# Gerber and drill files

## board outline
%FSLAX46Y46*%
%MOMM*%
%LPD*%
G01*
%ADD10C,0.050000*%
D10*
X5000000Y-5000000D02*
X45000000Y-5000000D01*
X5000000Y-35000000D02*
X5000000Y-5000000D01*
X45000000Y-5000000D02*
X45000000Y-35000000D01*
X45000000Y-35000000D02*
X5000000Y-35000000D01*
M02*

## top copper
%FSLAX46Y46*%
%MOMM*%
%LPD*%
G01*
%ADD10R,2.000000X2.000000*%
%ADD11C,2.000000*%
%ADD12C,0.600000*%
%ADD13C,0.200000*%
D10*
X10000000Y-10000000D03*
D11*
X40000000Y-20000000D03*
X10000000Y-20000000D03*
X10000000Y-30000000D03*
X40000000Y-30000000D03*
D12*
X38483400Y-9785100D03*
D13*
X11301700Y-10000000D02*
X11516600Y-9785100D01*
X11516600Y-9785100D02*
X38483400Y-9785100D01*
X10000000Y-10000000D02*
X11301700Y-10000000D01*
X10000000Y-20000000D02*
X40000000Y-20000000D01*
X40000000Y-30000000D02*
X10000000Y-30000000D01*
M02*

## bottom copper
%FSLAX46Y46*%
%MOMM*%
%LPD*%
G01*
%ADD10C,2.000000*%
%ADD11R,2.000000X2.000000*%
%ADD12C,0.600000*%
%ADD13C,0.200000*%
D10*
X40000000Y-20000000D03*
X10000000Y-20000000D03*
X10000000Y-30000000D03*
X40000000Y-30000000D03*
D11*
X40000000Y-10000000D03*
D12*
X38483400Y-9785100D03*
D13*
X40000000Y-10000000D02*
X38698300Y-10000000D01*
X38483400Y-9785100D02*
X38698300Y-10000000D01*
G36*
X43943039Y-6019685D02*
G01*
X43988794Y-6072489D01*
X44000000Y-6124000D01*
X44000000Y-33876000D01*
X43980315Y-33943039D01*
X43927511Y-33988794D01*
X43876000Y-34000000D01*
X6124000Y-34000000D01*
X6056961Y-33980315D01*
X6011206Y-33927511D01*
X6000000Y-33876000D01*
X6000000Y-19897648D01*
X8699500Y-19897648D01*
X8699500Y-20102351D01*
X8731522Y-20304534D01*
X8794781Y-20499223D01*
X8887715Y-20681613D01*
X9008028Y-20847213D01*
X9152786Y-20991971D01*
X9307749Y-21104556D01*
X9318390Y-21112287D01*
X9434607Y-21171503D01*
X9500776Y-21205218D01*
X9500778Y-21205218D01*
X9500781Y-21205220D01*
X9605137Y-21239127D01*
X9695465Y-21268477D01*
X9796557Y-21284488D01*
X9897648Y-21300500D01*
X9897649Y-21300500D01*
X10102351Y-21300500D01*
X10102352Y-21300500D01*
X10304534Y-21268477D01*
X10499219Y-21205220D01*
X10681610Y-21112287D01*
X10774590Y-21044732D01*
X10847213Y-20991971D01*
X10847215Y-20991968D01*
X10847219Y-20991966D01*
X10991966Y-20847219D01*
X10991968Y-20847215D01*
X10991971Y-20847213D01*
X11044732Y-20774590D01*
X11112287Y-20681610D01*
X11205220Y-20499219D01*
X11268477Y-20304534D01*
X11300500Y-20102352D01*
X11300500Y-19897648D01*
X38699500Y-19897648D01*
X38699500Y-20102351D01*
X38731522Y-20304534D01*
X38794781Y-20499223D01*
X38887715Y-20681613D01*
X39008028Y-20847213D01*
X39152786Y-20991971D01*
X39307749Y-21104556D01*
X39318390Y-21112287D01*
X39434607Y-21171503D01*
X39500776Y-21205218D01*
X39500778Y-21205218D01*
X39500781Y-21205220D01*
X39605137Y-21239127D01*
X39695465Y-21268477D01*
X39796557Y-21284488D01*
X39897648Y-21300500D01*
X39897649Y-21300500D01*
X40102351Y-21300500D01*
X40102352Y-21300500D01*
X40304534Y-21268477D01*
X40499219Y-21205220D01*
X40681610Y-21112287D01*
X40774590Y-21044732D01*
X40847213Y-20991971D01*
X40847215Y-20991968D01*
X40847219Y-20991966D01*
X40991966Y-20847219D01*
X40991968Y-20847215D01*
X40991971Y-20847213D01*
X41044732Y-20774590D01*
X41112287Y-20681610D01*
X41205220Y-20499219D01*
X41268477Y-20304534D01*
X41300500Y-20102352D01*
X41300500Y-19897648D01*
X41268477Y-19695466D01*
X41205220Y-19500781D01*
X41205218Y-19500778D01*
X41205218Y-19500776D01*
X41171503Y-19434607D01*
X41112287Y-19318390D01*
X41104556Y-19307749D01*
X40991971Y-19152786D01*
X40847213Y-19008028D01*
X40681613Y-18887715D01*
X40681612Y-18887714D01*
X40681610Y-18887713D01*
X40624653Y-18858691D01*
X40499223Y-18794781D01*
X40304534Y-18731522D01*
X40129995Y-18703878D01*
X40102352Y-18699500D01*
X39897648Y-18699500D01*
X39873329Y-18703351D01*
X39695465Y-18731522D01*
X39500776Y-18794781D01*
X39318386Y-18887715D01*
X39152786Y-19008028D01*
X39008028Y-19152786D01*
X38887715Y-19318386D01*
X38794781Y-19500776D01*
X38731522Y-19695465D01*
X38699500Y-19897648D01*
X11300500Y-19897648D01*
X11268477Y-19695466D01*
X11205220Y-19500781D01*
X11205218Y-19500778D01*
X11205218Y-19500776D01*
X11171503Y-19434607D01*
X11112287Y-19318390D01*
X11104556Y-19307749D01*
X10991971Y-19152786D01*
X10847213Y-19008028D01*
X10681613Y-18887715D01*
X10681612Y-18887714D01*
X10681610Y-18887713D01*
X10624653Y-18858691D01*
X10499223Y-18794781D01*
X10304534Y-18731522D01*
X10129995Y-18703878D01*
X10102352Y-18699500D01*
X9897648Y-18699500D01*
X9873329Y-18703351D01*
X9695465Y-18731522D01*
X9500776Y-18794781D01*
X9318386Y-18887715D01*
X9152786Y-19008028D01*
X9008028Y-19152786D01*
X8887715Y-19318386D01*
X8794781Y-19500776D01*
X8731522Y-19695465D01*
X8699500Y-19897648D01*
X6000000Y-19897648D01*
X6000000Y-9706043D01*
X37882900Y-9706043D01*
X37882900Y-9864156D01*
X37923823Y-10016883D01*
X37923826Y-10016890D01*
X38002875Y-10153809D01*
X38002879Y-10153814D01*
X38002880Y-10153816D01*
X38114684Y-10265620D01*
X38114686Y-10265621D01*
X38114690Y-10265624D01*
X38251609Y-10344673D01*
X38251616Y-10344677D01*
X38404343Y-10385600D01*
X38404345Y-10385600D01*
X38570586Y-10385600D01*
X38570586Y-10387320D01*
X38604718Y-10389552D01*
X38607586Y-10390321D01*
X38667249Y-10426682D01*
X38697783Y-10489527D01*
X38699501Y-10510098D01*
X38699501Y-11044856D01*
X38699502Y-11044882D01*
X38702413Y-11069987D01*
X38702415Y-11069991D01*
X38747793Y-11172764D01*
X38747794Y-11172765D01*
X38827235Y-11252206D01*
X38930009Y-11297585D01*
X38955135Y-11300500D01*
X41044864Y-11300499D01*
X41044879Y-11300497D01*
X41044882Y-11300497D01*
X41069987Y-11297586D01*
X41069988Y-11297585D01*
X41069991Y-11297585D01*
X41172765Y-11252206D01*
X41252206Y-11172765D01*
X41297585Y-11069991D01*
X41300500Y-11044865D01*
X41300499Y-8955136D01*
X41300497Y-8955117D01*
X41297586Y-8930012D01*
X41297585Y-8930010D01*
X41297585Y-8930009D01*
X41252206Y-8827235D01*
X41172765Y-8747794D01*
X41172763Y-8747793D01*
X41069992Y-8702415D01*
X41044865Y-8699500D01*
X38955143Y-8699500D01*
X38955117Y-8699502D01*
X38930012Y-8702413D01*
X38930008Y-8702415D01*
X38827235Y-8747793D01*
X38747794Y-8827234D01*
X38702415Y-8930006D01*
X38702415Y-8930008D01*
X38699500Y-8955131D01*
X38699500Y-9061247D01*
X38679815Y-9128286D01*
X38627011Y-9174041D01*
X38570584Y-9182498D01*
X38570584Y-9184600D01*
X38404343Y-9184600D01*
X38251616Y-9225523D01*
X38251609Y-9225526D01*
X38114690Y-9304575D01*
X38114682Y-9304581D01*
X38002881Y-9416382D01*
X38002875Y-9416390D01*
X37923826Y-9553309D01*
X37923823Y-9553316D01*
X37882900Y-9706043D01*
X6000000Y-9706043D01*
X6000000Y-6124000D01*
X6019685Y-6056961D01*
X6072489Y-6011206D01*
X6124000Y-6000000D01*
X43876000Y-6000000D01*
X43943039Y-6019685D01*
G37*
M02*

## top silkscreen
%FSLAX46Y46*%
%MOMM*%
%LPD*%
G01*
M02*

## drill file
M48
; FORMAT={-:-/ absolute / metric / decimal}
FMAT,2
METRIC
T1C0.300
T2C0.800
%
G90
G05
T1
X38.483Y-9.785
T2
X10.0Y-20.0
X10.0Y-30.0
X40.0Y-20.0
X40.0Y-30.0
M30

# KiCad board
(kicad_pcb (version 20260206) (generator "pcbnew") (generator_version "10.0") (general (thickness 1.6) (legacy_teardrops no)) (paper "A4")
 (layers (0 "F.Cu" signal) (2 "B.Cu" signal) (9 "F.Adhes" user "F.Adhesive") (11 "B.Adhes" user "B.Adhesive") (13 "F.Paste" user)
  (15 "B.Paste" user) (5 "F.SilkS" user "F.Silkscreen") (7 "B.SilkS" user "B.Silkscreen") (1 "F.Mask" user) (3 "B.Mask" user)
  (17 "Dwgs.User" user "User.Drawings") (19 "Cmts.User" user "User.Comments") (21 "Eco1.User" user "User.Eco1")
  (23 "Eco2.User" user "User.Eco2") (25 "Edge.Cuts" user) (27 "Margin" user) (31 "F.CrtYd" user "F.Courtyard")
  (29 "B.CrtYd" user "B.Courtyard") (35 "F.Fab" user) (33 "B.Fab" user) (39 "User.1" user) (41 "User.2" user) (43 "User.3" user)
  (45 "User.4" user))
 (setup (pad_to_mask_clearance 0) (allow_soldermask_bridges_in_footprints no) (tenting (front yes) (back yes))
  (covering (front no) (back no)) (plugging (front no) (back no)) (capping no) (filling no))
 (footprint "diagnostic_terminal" (layer "F.Cu") (at 10 10)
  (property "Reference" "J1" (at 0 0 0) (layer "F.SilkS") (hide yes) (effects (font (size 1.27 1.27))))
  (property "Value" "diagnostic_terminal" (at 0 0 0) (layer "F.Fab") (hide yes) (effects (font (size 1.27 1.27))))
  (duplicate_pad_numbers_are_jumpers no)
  (pad "1" smd rect (at 0 0) (size 2 2) (layers "F.Cu") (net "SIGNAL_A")))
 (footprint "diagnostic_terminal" (layer "F.Cu") (at 40 20)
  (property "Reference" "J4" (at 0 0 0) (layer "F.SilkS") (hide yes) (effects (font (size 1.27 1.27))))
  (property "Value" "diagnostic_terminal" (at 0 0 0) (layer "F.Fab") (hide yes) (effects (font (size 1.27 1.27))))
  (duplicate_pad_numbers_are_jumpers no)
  (pad "1" thru_hole circle (at 0 0) (size 2 2) (drill 0.8) (layers "*.Cu") (remove_unused_layers no) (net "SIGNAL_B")))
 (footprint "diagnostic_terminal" (layer "F.Cu") (at 10 20)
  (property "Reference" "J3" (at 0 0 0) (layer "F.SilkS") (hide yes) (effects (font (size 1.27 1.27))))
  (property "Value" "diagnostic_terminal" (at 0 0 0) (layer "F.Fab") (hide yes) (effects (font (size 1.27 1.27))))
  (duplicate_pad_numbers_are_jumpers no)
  (pad "1" thru_hole circle (at 0 0) (size 2 2) (drill 0.8) (layers "*.Cu") (remove_unused_layers no) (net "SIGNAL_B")))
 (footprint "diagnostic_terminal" (layer "F.Cu") (at 10 30)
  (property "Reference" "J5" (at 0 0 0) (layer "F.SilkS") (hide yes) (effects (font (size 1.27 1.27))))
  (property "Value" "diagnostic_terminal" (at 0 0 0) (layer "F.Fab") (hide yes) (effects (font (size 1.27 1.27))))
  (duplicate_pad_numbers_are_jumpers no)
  (pad "1" thru_hole circle (at 0 0) (size 2 2) (drill 0.8) (layers "*.Cu") (remove_unused_layers no) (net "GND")))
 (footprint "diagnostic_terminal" (layer "F.Cu") (at 40 30)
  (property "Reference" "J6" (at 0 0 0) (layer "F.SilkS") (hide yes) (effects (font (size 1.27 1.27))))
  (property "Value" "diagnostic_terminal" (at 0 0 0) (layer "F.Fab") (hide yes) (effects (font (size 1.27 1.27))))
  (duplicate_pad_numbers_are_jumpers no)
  (pad "1" thru_hole circle (at 0 0) (size 2 2) (drill 0.8) (layers "*.Cu") (remove_unused_layers no) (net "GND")))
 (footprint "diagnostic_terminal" (layer "B.Cu") (at 40 10)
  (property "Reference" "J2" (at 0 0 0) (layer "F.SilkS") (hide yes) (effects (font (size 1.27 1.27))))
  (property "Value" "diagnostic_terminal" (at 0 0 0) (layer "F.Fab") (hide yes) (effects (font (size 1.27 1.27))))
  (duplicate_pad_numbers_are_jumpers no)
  (pad "1" smd rect (at 0 0) (size 2 2) (layers "B.Cu") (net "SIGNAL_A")))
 (gr_line (start 5 5) (end 45 5) (stroke (width 0.05) (type default)) (layer "Edge.Cuts"))
 (gr_line (start 5 35) (end 5 5) (stroke (width 0.05) (type default)) (layer "Edge.Cuts"))
 (gr_line (start 45 5) (end 45 35) (stroke (width 0.05) (type default)) (layer "Edge.Cuts"))
 (gr_line (start 45 35) (end 5 35) (stroke (width 0.05) (type default)) (layer "Edge.Cuts"))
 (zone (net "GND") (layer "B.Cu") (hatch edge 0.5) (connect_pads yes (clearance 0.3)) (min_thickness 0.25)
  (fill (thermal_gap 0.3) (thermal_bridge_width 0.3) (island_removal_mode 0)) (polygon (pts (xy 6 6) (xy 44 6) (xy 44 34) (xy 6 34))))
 (segment (start 11.3017 10) (end 11.5166 9.7851) (width 0.2) (layer "F.Cu") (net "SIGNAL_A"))
 (segment (start 11.5166 9.7851) (end 38.4834 9.7851) (width 0.2) (layer "F.Cu") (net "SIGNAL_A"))
 (segment (start 10 10) (end 11.3017 10) (width 0.2) (layer "F.Cu") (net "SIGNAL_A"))
 (via (at 38.4834 9.7851) (size 0.6) (drill 0.3) (layers "F.Cu" "B.Cu") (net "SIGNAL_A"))
 (segment (start 40 10) (end 38.6983 10) (width 0.2) (layer "B.Cu") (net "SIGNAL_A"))
 (segment (start 38.4834 9.7851) (end 38.6983 10) (width 0.2) (layer "B.Cu") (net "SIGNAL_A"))
 (segment (start 10 20) (end 40 20) (width 0.2) (layer "F.Cu") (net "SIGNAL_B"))
 (segment (start 40 30) (end 10 30) (width 0.2) (layer "F.Cu") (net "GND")))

